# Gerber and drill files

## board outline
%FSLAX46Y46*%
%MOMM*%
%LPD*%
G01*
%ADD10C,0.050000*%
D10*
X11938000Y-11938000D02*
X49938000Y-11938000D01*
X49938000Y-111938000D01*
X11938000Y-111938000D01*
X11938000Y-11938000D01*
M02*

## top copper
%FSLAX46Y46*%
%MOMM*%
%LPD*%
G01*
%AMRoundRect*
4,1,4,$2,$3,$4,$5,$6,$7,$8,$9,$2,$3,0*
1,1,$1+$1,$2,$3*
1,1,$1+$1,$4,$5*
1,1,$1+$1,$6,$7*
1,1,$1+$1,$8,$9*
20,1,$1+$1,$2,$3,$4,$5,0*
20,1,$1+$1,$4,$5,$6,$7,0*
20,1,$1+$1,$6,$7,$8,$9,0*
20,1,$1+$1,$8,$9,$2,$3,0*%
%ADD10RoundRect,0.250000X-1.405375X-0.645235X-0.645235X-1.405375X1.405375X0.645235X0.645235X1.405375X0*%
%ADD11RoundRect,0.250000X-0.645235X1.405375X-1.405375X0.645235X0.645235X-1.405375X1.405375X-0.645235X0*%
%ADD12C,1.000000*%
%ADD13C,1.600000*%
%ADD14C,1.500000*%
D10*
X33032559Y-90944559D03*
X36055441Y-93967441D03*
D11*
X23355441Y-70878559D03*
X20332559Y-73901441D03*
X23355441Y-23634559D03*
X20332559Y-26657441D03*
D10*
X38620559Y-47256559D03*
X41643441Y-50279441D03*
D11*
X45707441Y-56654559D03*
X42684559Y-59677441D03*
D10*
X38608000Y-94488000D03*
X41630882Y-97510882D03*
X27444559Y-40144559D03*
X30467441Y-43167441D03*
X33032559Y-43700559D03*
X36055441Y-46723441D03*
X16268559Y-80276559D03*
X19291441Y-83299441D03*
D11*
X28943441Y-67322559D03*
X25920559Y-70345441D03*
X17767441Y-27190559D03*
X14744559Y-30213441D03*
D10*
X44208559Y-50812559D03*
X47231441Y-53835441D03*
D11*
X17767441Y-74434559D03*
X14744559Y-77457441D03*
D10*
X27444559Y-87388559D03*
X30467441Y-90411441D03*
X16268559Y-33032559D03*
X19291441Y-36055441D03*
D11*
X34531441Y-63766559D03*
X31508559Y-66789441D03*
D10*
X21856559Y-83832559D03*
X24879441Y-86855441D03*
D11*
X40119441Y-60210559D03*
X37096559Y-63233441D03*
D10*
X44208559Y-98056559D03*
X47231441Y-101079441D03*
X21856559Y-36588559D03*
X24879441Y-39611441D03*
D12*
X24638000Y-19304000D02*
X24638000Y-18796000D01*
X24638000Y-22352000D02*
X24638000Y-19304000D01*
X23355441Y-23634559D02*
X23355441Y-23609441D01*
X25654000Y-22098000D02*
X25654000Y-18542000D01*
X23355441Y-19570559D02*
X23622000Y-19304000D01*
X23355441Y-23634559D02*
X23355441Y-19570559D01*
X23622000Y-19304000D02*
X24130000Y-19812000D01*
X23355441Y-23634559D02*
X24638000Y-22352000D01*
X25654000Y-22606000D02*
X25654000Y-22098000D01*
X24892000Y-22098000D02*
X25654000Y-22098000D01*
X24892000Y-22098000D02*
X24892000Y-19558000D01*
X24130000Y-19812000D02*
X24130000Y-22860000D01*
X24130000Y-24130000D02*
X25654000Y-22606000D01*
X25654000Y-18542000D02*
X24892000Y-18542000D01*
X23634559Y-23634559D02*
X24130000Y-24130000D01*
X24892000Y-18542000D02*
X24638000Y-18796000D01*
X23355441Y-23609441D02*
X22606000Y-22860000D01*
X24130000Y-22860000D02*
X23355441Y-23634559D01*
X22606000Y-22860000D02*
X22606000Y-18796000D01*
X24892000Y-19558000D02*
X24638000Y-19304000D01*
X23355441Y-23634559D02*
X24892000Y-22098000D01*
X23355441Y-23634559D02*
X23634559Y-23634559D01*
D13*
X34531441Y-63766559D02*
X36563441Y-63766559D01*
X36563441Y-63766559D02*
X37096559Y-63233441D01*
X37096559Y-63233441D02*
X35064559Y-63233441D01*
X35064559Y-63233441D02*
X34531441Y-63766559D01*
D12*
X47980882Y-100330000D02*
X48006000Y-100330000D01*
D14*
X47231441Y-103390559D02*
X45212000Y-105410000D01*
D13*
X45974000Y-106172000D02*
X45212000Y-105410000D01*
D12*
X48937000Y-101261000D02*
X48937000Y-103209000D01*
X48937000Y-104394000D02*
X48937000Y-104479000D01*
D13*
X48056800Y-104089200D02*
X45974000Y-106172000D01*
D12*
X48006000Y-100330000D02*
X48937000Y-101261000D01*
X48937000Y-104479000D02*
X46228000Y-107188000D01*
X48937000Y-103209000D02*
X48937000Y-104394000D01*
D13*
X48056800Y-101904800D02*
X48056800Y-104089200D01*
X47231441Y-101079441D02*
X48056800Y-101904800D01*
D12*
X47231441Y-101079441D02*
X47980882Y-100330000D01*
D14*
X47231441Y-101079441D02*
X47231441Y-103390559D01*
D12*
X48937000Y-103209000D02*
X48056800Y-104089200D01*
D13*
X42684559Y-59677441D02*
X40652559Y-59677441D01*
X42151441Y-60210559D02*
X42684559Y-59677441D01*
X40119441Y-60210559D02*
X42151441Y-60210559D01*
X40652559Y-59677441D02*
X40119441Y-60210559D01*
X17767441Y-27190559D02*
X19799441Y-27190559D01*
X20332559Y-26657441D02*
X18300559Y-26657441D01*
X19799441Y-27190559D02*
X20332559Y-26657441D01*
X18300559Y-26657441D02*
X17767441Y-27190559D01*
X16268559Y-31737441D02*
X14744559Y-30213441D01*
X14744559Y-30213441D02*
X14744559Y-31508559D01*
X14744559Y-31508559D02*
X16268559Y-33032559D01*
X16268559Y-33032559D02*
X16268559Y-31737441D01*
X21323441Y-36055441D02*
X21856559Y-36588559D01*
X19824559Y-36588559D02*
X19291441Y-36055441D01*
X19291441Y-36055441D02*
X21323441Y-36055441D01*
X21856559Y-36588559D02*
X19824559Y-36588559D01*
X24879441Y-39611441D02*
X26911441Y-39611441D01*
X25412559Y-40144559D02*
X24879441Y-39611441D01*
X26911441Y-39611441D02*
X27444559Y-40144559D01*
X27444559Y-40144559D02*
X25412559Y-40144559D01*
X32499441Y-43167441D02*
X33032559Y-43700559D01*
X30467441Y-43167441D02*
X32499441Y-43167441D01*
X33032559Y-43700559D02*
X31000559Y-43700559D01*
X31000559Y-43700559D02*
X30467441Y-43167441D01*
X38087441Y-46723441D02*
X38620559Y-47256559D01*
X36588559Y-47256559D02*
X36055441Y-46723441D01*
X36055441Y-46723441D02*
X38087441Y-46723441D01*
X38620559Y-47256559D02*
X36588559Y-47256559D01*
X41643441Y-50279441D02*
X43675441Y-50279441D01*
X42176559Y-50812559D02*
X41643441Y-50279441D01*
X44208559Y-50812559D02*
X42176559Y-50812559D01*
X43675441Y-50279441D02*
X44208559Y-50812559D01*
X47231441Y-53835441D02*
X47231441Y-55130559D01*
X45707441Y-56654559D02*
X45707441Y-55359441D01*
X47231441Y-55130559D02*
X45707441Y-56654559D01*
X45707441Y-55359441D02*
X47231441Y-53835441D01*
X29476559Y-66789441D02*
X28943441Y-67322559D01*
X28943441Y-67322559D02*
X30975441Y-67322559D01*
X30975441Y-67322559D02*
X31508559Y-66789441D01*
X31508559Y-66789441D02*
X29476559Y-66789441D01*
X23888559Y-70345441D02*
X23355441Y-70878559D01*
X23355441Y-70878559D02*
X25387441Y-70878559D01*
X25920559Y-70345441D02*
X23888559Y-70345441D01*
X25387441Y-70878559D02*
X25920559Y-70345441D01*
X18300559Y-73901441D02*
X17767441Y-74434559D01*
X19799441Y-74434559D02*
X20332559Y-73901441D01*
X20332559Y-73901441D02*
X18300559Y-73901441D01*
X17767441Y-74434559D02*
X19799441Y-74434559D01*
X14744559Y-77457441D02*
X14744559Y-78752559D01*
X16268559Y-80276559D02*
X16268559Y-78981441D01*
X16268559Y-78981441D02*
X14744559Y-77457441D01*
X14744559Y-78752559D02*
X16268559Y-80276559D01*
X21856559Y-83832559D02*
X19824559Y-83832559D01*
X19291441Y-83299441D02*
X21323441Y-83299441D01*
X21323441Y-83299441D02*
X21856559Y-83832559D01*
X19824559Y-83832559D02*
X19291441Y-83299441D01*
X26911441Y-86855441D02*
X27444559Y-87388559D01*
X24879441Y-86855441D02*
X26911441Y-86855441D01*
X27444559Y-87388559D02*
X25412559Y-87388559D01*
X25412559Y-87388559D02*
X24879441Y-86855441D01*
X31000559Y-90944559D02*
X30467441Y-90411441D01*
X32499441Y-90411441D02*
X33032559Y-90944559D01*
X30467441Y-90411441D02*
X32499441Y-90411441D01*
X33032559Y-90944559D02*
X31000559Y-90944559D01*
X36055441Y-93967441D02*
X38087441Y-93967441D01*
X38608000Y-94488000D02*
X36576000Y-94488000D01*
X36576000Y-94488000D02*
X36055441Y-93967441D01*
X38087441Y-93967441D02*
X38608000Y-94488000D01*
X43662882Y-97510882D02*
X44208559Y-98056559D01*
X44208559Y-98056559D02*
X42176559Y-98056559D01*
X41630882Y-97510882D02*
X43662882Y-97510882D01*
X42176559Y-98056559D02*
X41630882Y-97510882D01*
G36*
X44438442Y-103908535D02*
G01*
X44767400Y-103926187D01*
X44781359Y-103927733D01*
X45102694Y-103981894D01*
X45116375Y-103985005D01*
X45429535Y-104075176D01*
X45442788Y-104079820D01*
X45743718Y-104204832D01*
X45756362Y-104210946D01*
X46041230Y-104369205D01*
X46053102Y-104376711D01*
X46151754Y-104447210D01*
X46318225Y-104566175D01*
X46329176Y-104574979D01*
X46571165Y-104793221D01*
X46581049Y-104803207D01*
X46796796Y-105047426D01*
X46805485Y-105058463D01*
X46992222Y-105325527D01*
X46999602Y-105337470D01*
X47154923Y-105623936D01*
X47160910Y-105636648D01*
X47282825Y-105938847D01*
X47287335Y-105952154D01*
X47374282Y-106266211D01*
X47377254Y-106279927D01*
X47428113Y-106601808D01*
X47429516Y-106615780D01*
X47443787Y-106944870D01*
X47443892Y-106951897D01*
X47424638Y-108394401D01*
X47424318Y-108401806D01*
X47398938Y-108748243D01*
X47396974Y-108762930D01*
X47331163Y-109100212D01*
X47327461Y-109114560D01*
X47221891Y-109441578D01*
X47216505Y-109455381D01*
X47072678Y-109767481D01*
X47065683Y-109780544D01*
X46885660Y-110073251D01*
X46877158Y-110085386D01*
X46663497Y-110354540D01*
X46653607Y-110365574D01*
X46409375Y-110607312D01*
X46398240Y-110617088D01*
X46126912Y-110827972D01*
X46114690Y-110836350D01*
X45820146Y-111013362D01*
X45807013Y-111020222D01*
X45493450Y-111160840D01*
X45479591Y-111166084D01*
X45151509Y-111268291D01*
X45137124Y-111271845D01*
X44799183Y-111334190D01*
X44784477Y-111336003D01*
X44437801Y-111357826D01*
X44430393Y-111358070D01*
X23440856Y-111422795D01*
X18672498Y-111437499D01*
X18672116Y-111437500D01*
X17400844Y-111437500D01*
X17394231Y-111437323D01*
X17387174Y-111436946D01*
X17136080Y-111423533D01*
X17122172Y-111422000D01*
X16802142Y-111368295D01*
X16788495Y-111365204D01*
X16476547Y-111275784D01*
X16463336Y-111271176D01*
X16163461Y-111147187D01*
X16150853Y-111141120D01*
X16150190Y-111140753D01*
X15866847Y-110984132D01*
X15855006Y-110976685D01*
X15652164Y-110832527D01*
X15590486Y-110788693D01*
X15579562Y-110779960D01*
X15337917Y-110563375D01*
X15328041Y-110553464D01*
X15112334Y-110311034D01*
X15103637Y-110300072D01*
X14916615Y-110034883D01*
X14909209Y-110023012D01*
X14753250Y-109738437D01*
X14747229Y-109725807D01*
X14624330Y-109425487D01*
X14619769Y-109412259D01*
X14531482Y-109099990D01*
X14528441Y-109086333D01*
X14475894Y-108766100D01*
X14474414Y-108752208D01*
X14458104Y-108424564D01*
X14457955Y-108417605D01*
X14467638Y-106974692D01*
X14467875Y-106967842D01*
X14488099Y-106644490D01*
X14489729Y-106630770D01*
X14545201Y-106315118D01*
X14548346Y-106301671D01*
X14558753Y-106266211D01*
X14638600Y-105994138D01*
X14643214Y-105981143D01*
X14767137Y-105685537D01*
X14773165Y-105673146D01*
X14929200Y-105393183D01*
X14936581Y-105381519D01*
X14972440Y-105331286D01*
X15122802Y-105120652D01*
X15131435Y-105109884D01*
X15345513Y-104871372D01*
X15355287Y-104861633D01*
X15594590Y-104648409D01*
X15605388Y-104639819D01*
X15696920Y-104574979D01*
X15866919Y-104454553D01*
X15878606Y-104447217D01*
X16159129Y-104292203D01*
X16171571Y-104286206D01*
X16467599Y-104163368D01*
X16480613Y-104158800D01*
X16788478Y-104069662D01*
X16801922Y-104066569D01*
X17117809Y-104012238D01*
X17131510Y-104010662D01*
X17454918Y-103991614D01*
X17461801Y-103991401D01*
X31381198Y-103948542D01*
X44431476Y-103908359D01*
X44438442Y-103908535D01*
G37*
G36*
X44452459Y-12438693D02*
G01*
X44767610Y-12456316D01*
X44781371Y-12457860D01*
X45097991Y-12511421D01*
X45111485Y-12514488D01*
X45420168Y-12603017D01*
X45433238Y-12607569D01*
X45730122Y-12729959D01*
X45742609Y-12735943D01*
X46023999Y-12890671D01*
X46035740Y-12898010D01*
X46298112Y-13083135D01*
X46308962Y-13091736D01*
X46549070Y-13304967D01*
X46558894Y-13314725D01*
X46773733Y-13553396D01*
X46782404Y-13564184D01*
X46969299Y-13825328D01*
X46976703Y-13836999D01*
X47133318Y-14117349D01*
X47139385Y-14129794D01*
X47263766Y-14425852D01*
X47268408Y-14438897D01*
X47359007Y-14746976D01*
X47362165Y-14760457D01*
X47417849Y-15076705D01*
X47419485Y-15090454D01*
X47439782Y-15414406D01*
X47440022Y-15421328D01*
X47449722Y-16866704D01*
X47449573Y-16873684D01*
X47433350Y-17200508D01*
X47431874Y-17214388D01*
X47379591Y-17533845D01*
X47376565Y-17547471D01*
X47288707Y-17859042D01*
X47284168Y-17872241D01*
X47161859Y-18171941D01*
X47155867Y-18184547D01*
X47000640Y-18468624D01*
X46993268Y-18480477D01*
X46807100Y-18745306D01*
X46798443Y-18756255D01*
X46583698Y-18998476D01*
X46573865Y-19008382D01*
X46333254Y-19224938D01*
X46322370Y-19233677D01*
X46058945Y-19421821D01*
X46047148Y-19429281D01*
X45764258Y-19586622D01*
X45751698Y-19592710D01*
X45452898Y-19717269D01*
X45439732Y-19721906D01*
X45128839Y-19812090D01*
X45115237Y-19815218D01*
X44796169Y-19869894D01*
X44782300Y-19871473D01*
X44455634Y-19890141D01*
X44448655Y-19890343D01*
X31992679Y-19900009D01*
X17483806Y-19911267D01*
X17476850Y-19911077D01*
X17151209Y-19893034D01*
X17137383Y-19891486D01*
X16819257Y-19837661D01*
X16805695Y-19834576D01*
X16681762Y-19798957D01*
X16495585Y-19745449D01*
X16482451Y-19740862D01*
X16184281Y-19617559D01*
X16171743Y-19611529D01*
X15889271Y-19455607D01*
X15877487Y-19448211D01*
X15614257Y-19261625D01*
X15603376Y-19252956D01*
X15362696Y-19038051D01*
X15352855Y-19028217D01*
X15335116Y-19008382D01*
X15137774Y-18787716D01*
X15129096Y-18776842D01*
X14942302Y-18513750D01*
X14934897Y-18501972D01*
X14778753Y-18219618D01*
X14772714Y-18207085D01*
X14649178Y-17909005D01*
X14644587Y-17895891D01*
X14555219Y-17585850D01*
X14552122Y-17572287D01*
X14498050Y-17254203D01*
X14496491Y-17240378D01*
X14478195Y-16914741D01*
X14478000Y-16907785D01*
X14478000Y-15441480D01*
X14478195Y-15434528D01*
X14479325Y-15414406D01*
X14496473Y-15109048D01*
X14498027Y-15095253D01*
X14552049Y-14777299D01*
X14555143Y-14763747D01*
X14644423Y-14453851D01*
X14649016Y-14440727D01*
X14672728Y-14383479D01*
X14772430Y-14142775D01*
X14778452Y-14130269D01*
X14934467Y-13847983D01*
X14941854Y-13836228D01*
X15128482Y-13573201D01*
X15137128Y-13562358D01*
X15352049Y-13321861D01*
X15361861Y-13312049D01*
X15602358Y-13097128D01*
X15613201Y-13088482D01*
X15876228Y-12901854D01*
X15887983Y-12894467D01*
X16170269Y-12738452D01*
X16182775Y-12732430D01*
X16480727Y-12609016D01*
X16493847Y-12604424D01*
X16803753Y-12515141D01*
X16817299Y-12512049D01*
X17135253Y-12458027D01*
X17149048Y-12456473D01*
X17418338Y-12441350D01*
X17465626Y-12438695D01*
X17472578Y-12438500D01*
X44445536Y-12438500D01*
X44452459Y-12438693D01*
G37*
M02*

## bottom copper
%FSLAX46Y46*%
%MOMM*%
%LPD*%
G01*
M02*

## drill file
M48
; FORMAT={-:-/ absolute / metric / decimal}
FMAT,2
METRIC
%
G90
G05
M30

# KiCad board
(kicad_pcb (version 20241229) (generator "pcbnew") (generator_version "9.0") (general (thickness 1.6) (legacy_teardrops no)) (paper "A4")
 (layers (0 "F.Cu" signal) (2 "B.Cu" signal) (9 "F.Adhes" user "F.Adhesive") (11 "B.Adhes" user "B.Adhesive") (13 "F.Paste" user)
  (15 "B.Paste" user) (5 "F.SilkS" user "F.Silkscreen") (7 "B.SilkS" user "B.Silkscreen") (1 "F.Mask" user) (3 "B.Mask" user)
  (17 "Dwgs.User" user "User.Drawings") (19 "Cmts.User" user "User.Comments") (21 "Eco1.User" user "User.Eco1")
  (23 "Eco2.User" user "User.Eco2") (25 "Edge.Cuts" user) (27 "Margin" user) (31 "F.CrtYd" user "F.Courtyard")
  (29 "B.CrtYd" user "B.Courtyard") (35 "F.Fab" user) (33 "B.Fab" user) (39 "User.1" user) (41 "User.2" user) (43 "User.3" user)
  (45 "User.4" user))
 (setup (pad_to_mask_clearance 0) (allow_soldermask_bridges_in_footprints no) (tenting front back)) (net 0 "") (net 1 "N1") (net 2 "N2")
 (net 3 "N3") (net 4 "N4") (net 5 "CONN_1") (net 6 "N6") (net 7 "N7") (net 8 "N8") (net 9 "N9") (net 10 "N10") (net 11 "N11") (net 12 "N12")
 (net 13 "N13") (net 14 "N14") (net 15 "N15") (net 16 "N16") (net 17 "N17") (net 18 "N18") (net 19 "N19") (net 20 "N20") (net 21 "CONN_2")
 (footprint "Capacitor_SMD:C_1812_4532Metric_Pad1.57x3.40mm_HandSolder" (layer "F.Cu") (at 34.544 92.456 -45)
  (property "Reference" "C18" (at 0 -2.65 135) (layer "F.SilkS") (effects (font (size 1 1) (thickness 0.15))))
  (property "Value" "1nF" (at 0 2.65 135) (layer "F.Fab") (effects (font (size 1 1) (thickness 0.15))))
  (pad "1" smd roundrect (at -2.1375 0 315) (size 1.575 3.4) (layers "F.Cu" "F.Mask" "F.Paste") (roundrect_rratio 0.15873) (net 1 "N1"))
  (pad "2" smd roundrect (at 2.1375 0 315) (size 1.575 3.4) (layers "F.Cu" "F.Mask" "F.Paste") (roundrect_rratio 0.15873) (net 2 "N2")))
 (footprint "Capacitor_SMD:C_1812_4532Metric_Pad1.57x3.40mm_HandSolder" (layer "F.Cu") (at 21.844 72.39 -135)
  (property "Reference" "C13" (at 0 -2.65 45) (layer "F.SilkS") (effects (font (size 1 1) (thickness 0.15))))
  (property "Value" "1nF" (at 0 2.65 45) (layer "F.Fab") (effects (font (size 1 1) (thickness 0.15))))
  (pad "1" smd roundrect (at -2.1375 0 225) (size 1.575 3.4) (layers "F.Cu" "F.Mask" "F.Paste") (roundrect_rratio 0.15873) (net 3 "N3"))
  (pad "2" smd roundrect (at 2.1375 0 225) (size 1.575 3.4) (layers "F.Cu" "F.Mask" "F.Paste") (roundrect_rratio 0.15873) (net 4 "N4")))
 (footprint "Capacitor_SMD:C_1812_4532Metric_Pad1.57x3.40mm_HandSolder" (layer "F.Cu") (at 21.844 25.146 -135)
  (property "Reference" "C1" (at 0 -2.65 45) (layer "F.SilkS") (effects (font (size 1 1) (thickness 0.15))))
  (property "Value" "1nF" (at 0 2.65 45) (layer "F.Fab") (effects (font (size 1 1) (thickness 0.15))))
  (pad "1" smd roundrect (at -2.1375 0 225) (size 1.575 3.4) (layers "F.Cu" "F.Mask" "F.Paste") (roundrect_rratio 0.15873) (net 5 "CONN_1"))
  (pad "2" smd roundrect (at 2.1375 0 225) (size 1.575 3.4) (layers "F.Cu" "F.Mask" "F.Paste") (roundrect_rratio 0.15873) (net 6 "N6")))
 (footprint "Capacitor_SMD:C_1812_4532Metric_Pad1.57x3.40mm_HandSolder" (layer "F.Cu") (at 40.132 48.768 -45)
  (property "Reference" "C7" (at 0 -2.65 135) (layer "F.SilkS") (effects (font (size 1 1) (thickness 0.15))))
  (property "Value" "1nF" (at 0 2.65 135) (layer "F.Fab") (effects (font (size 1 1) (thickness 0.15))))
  (pad "1" smd roundrect (at -2.1375 0 315) (size 1.575 3.4) (layers "F.Cu" "F.Mask" "F.Paste") (roundrect_rratio 0.15873) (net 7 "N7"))
  (pad "2" smd roundrect (at 2.1375 0 315) (size 1.575 3.4) (layers "F.Cu" "F.Mask" "F.Paste") (roundrect_rratio 0.15873) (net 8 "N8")))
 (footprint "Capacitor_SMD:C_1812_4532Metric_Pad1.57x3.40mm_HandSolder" (layer "F.Cu") (at 44.196 58.166 -135)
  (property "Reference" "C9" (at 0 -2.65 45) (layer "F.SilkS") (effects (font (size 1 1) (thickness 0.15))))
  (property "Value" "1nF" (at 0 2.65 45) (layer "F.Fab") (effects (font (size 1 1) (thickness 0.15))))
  (pad "1" smd roundrect (at -2.1375 0 225) (size 1.575 3.4) (layers "F.Cu" "F.Mask" "F.Paste") (roundrect_rratio 0.15873) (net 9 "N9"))
  (pad "2" smd roundrect (at 2.1375 0 225) (size 1.575 3.4) (layers "F.Cu" "F.Mask" "F.Paste") (roundrect_rratio 0.15873) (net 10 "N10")))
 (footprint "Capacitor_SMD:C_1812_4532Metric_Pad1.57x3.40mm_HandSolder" (layer "F.Cu") (at 40.119441 95.999441 -45)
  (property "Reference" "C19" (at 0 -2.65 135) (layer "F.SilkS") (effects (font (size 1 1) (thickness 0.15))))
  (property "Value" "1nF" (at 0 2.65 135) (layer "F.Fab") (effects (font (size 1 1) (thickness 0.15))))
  (pad "1" smd roundrect (at -2.1375 0 315) (size 1.575 3.4) (layers "F.Cu" "F.Mask" "F.Paste") (roundrect_rratio 0.15873) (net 2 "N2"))
  (pad "2" smd roundrect (at 2.1375 0 315) (size 1.575 3.4) (layers "F.Cu" "F.Mask" "F.Paste") (roundrect_rratio 0.15873) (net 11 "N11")))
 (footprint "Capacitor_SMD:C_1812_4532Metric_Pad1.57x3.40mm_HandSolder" (layer "F.Cu") (at 28.956 41.656 -45)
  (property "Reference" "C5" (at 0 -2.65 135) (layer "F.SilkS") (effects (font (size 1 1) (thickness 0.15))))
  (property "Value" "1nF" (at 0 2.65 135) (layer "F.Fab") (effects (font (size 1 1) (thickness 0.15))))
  (pad "1" smd roundrect (at -2.1375 0 315) (size 1.575 3.4) (layers "F.Cu" "F.Mask" "F.Paste") (roundrect_rratio 0.15873) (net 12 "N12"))
  (pad "2" smd roundrect (at 2.1375 0 315) (size 1.575 3.4) (layers "F.Cu" "F.Mask" "F.Paste") (roundrect_rratio 0.15873) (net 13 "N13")))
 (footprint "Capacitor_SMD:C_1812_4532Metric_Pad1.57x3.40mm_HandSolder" (layer "F.Cu") (at 34.544 45.212 -45)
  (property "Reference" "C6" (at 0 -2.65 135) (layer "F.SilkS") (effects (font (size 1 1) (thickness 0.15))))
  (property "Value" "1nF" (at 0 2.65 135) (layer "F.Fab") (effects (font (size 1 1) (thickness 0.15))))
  (pad "1" smd roundrect (at -2.1375 0 315) (size 1.575 3.4) (layers "F.Cu" "F.Mask" "F.Paste") (roundrect_rratio 0.15873) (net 13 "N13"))
  (pad "2" smd roundrect (at 2.1375 0 315) (size 1.575 3.4) (layers "F.Cu" "F.Mask" "F.Paste") (roundrect_rratio 0.15873) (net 7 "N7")))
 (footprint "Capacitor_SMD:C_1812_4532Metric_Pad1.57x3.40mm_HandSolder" (layer "F.Cu") (at 17.78 81.788 -45)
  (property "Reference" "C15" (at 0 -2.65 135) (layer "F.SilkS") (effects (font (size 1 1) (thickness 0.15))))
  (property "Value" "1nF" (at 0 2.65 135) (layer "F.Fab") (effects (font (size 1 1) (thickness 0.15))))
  (pad "1" smd roundrect (at -2.1375 0 315) (size 1.575 3.4) (layers "F.Cu" "F.Mask" "F.Paste") (roundrect_rratio 0.15873) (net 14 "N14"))
  (pad "2" smd roundrect (at 2.1375 0 315) (size 1.575 3.4) (layers "F.Cu" "F.Mask" "F.Paste") (roundrect_rratio 0.15873) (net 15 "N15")))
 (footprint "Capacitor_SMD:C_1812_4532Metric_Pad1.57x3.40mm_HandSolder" (layer "F.Cu") (at 27.432 68.834 -135)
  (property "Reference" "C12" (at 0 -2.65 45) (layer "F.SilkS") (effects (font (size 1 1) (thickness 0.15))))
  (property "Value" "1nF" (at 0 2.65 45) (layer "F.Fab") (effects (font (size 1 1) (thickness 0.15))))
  (pad "1" smd roundrect (at -2.1375 0 225) (size 1.575 3.4) (layers "F.Cu" "F.Mask" "F.Paste") (roundrect_rratio 0.15873) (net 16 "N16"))
  (pad "2" smd roundrect (at 2.1375 0 225) (size 1.575 3.4) (layers "F.Cu" "F.Mask" "F.Paste") (roundrect_rratio 0.15873) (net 3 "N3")))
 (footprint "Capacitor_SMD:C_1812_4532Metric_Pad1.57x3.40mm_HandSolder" (layer "F.Cu") (at 16.256 28.702 -135)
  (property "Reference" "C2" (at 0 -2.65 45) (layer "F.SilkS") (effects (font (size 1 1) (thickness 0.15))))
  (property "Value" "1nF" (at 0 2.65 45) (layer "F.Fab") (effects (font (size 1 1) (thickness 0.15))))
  (pad "1" smd roundrect (at -2.1375 0 225) (size 1.575 3.4) (layers "F.Cu" "F.Mask" "F.Paste") (roundrect_rratio 0.15873) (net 6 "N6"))
  (pad "2" smd roundrect (at 2.1375 0 225) (size 1.575 3.4) (layers "F.Cu" "F.Mask" "F.Paste") (roundrect_rratio 0.15873) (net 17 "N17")))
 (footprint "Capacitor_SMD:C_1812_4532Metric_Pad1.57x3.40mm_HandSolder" (layer "F.Cu") (at 45.72 52.324 -45)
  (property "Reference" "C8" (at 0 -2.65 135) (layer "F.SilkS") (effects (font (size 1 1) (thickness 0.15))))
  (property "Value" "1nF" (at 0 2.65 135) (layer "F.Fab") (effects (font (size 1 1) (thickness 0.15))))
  (pad "1" smd roundrect (at -2.1375 0 315) (size 1.575 3.4) (layers "F.Cu" "F.Mask" "F.Paste") (roundrect_rratio 0.15873) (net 8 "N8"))
  (pad "2" smd roundrect (at 2.1375 0 315) (size 1.575 3.4) (layers "F.Cu" "F.Mask" "F.Paste") (roundrect_rratio 0.15873) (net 9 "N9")))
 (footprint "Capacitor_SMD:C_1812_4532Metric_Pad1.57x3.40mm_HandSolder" (layer "F.Cu") (at 16.256 75.946 -135)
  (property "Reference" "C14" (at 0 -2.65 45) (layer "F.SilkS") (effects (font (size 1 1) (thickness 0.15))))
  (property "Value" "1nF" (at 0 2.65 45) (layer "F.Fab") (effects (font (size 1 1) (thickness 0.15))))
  (pad "1" smd roundrect (at -2.1375 0 225) (size 1.575 3.4) (layers "F.Cu" "F.Mask" "F.Paste") (roundrect_rratio 0.15873) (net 4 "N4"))
  (pad "2" smd roundrect (at 2.1375 0 225) (size 1.575 3.4) (layers "F.Cu" "F.Mask" "F.Paste") (roundrect_rratio 0.15873) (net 14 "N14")))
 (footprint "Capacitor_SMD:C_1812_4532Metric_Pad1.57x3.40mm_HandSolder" (layer "F.Cu") (at 28.956 88.9 -45)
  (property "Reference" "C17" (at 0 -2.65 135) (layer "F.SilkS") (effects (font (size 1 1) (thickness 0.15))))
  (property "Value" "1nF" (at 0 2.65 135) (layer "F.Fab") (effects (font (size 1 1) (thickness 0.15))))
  (pad "1" smd roundrect (at -2.1375 0 315) (size 1.575 3.4) (layers "F.Cu" "F.Mask" "F.Paste") (roundrect_rratio 0.15873) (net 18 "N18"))
  (pad "2" smd roundrect (at 2.1375 0 315) (size 1.575 3.4) (layers "F.Cu" "F.Mask" "F.Paste") (roundrect_rratio 0.15873) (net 1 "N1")))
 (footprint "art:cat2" (layer "F.Cu") (at 22.606 55.372 45)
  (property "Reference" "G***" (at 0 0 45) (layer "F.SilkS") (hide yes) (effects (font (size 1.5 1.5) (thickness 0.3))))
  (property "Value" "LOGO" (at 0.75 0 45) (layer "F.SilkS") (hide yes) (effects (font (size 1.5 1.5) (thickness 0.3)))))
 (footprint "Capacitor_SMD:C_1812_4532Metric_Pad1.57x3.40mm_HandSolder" (layer "F.Cu") (at 17.78 34.544 -45)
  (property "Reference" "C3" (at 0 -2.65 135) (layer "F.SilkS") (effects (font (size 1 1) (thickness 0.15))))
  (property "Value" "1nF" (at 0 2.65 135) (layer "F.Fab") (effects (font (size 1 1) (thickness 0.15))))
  (pad "1" smd roundrect (at -2.1375 0 315) (size 1.575 3.4) (layers "F.Cu" "F.Mask" "F.Paste") (roundrect_rratio 0.15873) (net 17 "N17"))
  (pad "2" smd roundrect (at 2.1375 0 315) (size 1.575 3.4) (layers "F.Cu" "F.Mask" "F.Paste") (roundrect_rratio 0.15873) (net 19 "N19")))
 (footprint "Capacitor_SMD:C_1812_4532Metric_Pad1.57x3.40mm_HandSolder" (layer "F.Cu") (at 33.02 65.278 -135)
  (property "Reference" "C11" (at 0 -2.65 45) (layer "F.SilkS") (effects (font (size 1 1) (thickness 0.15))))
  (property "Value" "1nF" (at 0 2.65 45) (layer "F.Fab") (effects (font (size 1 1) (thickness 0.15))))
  (pad "1" smd roundrect (at -2.1375 0 225) (size 1.575 3.4) (layers "F.Cu" "F.Mask" "F.Paste") (roundrect_rratio 0.15873) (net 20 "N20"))
  (pad "2" smd roundrect (at 2.1375 0 225) (size 1.575 3.4) (layers "F.Cu" "F.Mask" "F.Paste") (roundrect_rratio 0.15873) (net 16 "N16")))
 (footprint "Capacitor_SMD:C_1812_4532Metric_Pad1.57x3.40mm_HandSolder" (layer "F.Cu") (at 23.368 85.344 -45)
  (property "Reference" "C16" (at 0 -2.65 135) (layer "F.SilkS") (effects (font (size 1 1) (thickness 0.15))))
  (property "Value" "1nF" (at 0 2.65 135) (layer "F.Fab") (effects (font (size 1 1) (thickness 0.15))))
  (pad "1" smd roundrect (at -2.1375 0 315) (size 1.575 3.4) (layers "F.Cu" "F.Mask" "F.Paste") (roundrect_rratio 0.15873) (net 15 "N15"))
  (pad "2" smd roundrect (at 2.1375 0 315) (size 1.575 3.4) (layers "F.Cu" "F.Mask" "F.Paste") (roundrect_rratio 0.15873) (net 18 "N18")))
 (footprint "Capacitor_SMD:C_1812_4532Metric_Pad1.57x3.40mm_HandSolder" (layer "F.Cu") (at 38.608 61.722 -135)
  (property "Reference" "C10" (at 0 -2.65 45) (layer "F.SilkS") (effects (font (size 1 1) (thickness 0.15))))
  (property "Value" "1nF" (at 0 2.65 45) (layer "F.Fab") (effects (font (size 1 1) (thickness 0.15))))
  (pad "1" smd roundrect (at -2.1375 0 225) (size 1.575 3.4) (layers "F.Cu" "F.Mask" "F.Paste") (roundrect_rratio 0.15873) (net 10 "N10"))
  (pad "2" smd roundrect (at 2.1375 0 225) (size 1.575 3.4) (layers "F.Cu" "F.Mask" "F.Paste") (roundrect_rratio 0.15873) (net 20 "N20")))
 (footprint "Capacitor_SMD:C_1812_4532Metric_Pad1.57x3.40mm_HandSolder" (layer "F.Cu") (at 45.72 99.568 -45)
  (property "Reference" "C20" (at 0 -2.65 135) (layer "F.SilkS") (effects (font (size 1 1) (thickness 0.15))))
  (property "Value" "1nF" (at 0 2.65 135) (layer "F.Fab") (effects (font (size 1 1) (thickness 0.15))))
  (pad "1" smd roundrect (at -2.1375 0 315) (size 1.575 3.4) (layers "F.Cu" "F.Mask" "F.Paste") (roundrect_rratio 0.15873) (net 11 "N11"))
  (pad "2" smd roundrect (at 2.1375 0 315) (size 1.575 3.4) (layers "F.Cu" "F.Mask" "F.Paste") (roundrect_rratio 0.15873) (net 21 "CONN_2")))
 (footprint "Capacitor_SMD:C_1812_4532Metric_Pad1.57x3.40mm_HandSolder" (layer "F.Cu") (at 23.368 38.1 -45)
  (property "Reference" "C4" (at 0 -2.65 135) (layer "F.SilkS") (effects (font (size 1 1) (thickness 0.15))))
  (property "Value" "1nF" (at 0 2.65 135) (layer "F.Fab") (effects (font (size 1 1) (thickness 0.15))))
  (pad "1" smd roundrect (at -2.1375 0 315) (size 1.575 3.4) (layers "F.Cu" "F.Mask" "F.Paste") (roundrect_rratio 0.15873) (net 19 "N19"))
  (pad "2" smd roundrect (at 2.1375 0 315) (size 1.575 3.4) (layers "F.Cu" "F.Mask" "F.Paste") (roundrect_rratio 0.15873) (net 12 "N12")))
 (gr_rect (start 11.938 11.938) (end 49.938 111.938) (stroke (width 0.05) (type solid)) (fill no) (layer "Edge.Cuts"))
 (segment (start 24.638 19.304) (end 24.638 18.796) (width 1) (layer "F.Cu") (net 5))
 (segment (start 24.638 22.352) (end 24.638 19.304) (width 1) (layer "F.Cu") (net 5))
 (segment (start 23.355441 23.634559) (end 23.355441 23.609441) (width 1) (layer "F.Cu") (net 5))
 (segment (start 25.654 22.098) (end 25.654 18.542) (width 1) (layer "F.Cu") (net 5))
 (segment (start 23.355441 19.570559) (end 23.622 19.304) (width 1) (layer "F.Cu") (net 5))
 (segment (start 23.355441 23.634559) (end 23.355441 19.570559) (width 1) (layer "F.Cu") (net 5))
 (segment (start 23.622 19.304) (end 24.13 19.812) (width 1) (layer "F.Cu") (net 5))
 (segment (start 23.355441 23.634559) (end 24.638 22.352) (width 1) (layer "F.Cu") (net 5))
 (segment (start 25.654 22.606) (end 25.654 22.098) (width 1) (layer "F.Cu") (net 5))
 (segment (start 24.892 22.098) (end 25.654 22.098) (width 1) (layer "F.Cu") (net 5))
 (segment (start 24.892 22.098) (end 24.892 19.558) (width 1) (layer "F.Cu") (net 5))
 (segment (start 24.13 19.812) (end 24.13 22.86) (width 1) (layer "F.Cu") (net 5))
 (segment (start 24.13 24.13) (end 25.654 22.606) (width 1) (layer "F.Cu") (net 5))
 (segment (start 25.654 18.542) (end 24.892 18.542) (width 1) (layer "F.Cu") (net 5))
 (segment (start 23.634559 23.634559) (end 24.13 24.13) (width 1) (layer "F.Cu") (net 5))
 (segment (start 24.892 18.542) (end 24.638 18.796) (width 1) (layer "F.Cu") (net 5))
 (segment (start 23.355441 23.609441) (end 22.606 22.86) (width 1) (layer "F.Cu") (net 5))
 (segment (start 24.13 22.86) (end 23.355441 23.634559) (width 1) (layer "F.Cu") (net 5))
 (segment (start 22.606 22.86) (end 22.606 18.796) (width 1) (layer "F.Cu") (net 5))
 (segment (start 24.892 19.558) (end 24.638 19.304) (width 1) (layer "F.Cu") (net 5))
 (segment (start 23.355441 23.634559) (end 24.892 22.098) (width 1) (layer "F.Cu") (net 5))
 (segment (start 23.355441 23.634559) (end 23.634559 23.634559) (width 1) (layer "F.Cu") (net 5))
 (segment (start 34.531441 63.766559) (end 36.563441 63.766559) (width 1.6) (layer "F.Cu") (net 20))
 (segment (start 36.563441 63.766559) (end 37.096559 63.233441) (width 1.6) (layer "F.Cu") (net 20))
 (segment (start 37.096559 63.233441) (end 35.064559 63.233441) (width 1.6) (layer "F.Cu") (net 20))
 (segment (start 35.064559 63.233441) (end 34.531441 63.766559) (width 1.6) (layer "F.Cu") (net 20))
 (segment (start 47.980882 100.33) (end 48.006 100.33) (width 1) (layer "F.Cu") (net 21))
 (segment (start 47.231441 103.390559) (end 45.212 105.41) (width 1.5) (layer "F.Cu") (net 21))
 (segment (start 45.974 106.172) (end 45.212 105.41) (width 1.6) (layer "F.Cu") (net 21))
 (segment (start 48.937 101.261) (end 48.937 103.209) (width 1) (layer "F.Cu") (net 21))
 (segment (start 48.937 104.394) (end 48.937 104.479) (width 1) (layer "F.Cu") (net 21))
 (segment (start 48.0568 104.0892) (end 45.974 106.172) (width 1.6) (layer "F.Cu") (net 21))
 (segment (start 48.006 100.33) (end 48.937 101.261) (width 1) (layer "F.Cu") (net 21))
 (segment (start 48.937 104.479) (end 46.228 107.188) (width 1) (layer "F.Cu") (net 21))
 (segment (start 48.937 103.209) (end 48.937 104.394) (width 1) (layer "F.Cu") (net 21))
 (segment (start 48.0568 101.9048) (end 48.0568 104.0892) (width 1.6) (layer "F.Cu") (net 21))
 (segment (start 47.231441 101.079441) (end 48.0568 101.9048) (width 1.6) (layer "F.Cu") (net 21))
 (segment (start 47.231441 101.079441) (end 47.980882 100.33) (width 1) (layer "F.Cu") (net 21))
 (segment (start 47.231441 101.079441) (end 47.231441 103.390559) (width 1.5) (layer "F.Cu") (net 21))
 (segment (start 48.937 103.209) (end 48.0568 104.0892) (width 1) (layer "F.Cu") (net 21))
 (segment (start 42.684559 59.677441) (end 40.652559 59.677441) (width 1.6) (layer "F.Cu") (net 10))
 (segment (start 42.151441 60.210559) (end 42.684559 59.677441) (width 1.6) (layer "F.Cu") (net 10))
 (segment (start 40.119441 60.210559) (end 42.151441 60.210559) (width 1.6) (layer "F.Cu") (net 10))
 (segment (start 40.652559 59.677441) (end 40.119441 60.210559) (width 1.6) (layer "F.Cu") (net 10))
 (segment (start 17.767441 27.190559) (end 19.799441 27.190559) (width 1.6) (layer "F.Cu") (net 6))
 (segment (start 20.332559 26.657441) (end 18.300559 26.657441) (width 1.6) (layer "F.Cu") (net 6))
 (segment (start 19.799441 27.190559) (end 20.332559 26.657441) (width 1.6) (layer "F.Cu") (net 6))
 (segment (start 18.300559 26.657441) (end 17.767441 27.190559) (width 1.6) (layer "F.Cu") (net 6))
 (segment (start 16.268559 31.737441) (end 14.744559 30.213441) (width 1.6) (layer "F.Cu") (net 17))
 (segment (start 14.744559 30.213441) (end 14.744559 31.508559) (width 1.6) (layer "F.Cu") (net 17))
 (segment (start 14.744559 31.508559) (end 16.268559 33.032559) (width 1.6) (layer "F.Cu") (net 17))
 (segment (start 16.268559 33.032559) (end 16.268559 31.737441) (width 1.6) (layer "F.Cu") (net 17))
 (segment (start 21.323441 36.055441) (end 21.856559 36.588559) (width 1.6) (layer "F.Cu") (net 19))
 (segment (start 19.824559 36.588559) (end 19.291441 36.055441) (width 1.6) (layer "F.Cu") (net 19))
 (segment (start 19.291441 36.055441) (end 21.323441 36.055441) (width 1.6) (layer "F.Cu") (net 19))
 (segment (start 21.856559 36.588559) (end 19.824559 36.588559) (width 1.6) (layer "F.Cu") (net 19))
 (segment (start 24.879441 39.611441) (end 26.911441 39.611441) (width 1.6) (layer "F.Cu") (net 12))
 (segment (start 25.412559 40.144559) (end 24.879441 39.611441) (width 1.6) (layer "F.Cu") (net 12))
 (segment (start 26.911441 39.611441) (end 27.444559 40.144559) (width 1.6) (layer "F.Cu") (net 12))
 (segment (start 27.444559 40.144559) (end 25.412559 40.144559) (width 1.6) (layer "F.Cu") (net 12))
 (segment (start 32.499441 43.167441) (end 33.032559 43.700559) (width 1.6) (layer "F.Cu") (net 13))
 (segment (start 30.467441 43.167441) (end 32.499441 43.167441) (width 1.6) (layer "F.Cu") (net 13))
 (segment (start 33.032559 43.700559) (end 31.000559 43.700559) (width 1.6) (layer "F.Cu") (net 13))
 (segment (start 31.000559 43.700559) (end 30.467441 43.167441) (width 1.6) (layer "F.Cu") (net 13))
 (segment (start 38.087441 46.723441) (end 38.620559 47.256559) (width 1.6) (layer "F.Cu") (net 7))
 (segment (start 36.588559 47.256559) (end 36.055441 46.723441) (width 1.6) (layer "F.Cu") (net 7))
 (segment (start 36.055441 46.723441) (end 38.087441 46.723441) (width 1.6) (layer "F.Cu") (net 7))
 (segment (start 38.620559 47.256559) (end 36.588559 47.256559) (width 1.6) (layer "F.Cu") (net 7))
 (segment (start 41.643441 50.279441) (end 43.675441 50.279441) (width 1.6) (layer "F.Cu") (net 8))
 (segment (start 42.176559 50.812559) (end 41.643441 50.279441) (width 1.6) (layer "F.Cu") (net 8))
 (segment (start 44.208559 50.812559) (end 42.176559 50.812559) (width 1.6) (layer "F.Cu") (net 8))
 (segment (start 43.675441 50.279441) (end 44.208559 50.812559) (width 1.6) (layer "F.Cu") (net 8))
 (segment (start 47.231441 53.835441) (end 47.231441 55.130559) (width 1.6) (layer "F.Cu") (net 9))
 (segment (start 45.707441 56.654559) (end 45.707441 55.359441) (width 1.6) (layer "F.Cu") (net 9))
 (segment (start 47.231441 55.130559) (end 45.707441 56.654559) (width 1.6) (layer "F.Cu") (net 9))
 (segment (start 45.707441 55.359441) (end 47.231441 53.835441) (width 1.6) (layer "F.Cu") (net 9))
 (segment (start 29.476559 66.789441) (end 28.943441 67.322559) (width 1.6) (layer "F.Cu") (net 16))
 (segment (start 28.943441 67.322559) (end 30.975441 67.322559) (width 1.6) (layer "F.Cu") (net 16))
 (segment (start 30.975441 67.322559) (end 31.508559 66.789441) (width 1.6) (layer "F.Cu") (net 16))
 (segment (start 31.508559 66.789441) (end 29.476559 66.789441) (width 1.6) (layer "F.Cu") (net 16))
 (segment (start 23.888559 70.345441) (end 23.355441 70.878559) (width 1.6) (layer "F.Cu") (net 3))
 (segment (start 23.355441 70.878559) (end 25.387441 70.878559) (width 1.6) (layer "F.Cu") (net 3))
 (segment (start 25.920559 70.345441) (end 23.888559 70.345441) (width 1.6) (layer "F.Cu") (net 3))
 (segment (start 25.387441 70.878559) (end 25.920559 70.345441) (width 1.6) (layer "F.Cu") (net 3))
 (segment (start 18.300559 73.901441) (end 17.767441 74.434559) (width 1.6) (layer "F.Cu") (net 4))
 (segment (start 19.799441 74.434559) (end 20.332559 73.901441) (width 1.6) (layer "F.Cu") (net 4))
 (segment (start 20.332559 73.901441) (end 18.300559 73.901441) (width 1.6) (layer "F.Cu") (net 4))
 (segment (start 17.767441 74.434559) (end 19.799441 74.434559) (width 1.6) (layer "F.Cu") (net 4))
 (segment (start 14.744559 77.457441) (end 14.744559 78.752559) (width 1.6) (layer "F.Cu") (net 14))
 (segment (start 16.268559 80.276559) (end 16.268559 78.981441) (width 1.6) (layer "F.Cu") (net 14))
 (segment (start 16.268559 78.981441) (end 14.744559 77.457441) (width 1.6) (layer "F.Cu") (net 14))
 (segment (start 14.744559 78.752559) (end 16.268559 80.276559) (width 1.6) (layer "F.Cu") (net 14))
 (segment (start 21.856559 83.832559) (end 19.824559 83.832559) (width 1.6) (layer "F.Cu") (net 15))
 (segment (start 19.291441 83.299441) (end 21.323441 83.299441) (width 1.6) (layer "F.Cu") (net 15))
 (segment (start 21.323441 83.299441) (end 21.856559 83.832559) (width 1.6) (layer "F.Cu") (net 15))
 (segment (start 19.824559 83.832559) (end 19.291441 83.299441) (width 1.6) (layer "F.Cu") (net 15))
 (segment (start 26.911441 86.855441) (end 27.444559 87.388559) (width 1.6) (layer "F.Cu") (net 18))
 (segment (start 24.879441 86.855441) (end 26.911441 86.855441) (width 1.6) (layer "F.Cu") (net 18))
 (segment (start 27.444559 87.388559) (end 25.412559 87.388559) (width 1.6) (layer "F.Cu") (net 18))
 (segment (start 25.412559 87.388559) (end 24.879441 86.855441) (width 1.6) (layer "F.Cu") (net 18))
 (segment (start 31.000559 90.944559) (end 30.467441 90.411441) (width 1.6) (layer "F.Cu") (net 1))
 (segment (start 32.499441 90.411441) (end 33.032559 90.944559) (width 1.6) (layer "F.Cu") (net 1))
 (segment (start 30.467441 90.411441) (end 32.499441 90.411441) (width 1.6) (layer "F.Cu") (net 1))
 (segment (start 33.032559 90.944559) (end 31.000559 90.944559) (width 1.6) (layer "F.Cu") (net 1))
 (segment (start 36.055441 93.967441) (end 38.087441 93.967441) (width 1.6) (layer "F.Cu") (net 2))
 (segment (start 38.608 94.488) (end 36.576 94.488) (width 1.6) (layer "F.Cu") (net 2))
 (segment (start 36.576 94.488) (end 36.055441 93.967441) (width 1.6) (layer "F.Cu") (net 2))
 (segment (start 38.087441 93.967441) (end 38.608 94.488) (width 1.6) (layer "F.Cu") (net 2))
 (segment (start 43.662882 97.510882) (end 44.208559 98.056559) (width 1.6) (layer "F.Cu") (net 11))
 (segment (start 44.208559 98.056559) (end 42.176559 98.056559) (width 1.6) (layer "F.Cu") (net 11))
 (segment (start 41.630882 97.510882) (end 43.662882 97.510882) (width 1.6) (layer "F.Cu") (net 11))
 (segment (start 42.176559 98.056559) (end 41.630882 97.510882) (width 1.6) (layer "F.Cu") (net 11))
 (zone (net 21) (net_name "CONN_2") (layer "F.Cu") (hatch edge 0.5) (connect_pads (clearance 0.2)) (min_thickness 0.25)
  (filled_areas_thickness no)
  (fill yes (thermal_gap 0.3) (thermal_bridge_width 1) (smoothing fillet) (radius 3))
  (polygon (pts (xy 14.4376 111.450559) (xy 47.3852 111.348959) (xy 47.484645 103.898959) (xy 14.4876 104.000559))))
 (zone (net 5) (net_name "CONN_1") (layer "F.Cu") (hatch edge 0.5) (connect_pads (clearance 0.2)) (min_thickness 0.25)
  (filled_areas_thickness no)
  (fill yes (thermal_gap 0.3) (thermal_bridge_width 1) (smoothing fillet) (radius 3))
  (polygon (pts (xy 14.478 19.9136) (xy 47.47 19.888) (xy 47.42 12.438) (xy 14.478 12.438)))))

